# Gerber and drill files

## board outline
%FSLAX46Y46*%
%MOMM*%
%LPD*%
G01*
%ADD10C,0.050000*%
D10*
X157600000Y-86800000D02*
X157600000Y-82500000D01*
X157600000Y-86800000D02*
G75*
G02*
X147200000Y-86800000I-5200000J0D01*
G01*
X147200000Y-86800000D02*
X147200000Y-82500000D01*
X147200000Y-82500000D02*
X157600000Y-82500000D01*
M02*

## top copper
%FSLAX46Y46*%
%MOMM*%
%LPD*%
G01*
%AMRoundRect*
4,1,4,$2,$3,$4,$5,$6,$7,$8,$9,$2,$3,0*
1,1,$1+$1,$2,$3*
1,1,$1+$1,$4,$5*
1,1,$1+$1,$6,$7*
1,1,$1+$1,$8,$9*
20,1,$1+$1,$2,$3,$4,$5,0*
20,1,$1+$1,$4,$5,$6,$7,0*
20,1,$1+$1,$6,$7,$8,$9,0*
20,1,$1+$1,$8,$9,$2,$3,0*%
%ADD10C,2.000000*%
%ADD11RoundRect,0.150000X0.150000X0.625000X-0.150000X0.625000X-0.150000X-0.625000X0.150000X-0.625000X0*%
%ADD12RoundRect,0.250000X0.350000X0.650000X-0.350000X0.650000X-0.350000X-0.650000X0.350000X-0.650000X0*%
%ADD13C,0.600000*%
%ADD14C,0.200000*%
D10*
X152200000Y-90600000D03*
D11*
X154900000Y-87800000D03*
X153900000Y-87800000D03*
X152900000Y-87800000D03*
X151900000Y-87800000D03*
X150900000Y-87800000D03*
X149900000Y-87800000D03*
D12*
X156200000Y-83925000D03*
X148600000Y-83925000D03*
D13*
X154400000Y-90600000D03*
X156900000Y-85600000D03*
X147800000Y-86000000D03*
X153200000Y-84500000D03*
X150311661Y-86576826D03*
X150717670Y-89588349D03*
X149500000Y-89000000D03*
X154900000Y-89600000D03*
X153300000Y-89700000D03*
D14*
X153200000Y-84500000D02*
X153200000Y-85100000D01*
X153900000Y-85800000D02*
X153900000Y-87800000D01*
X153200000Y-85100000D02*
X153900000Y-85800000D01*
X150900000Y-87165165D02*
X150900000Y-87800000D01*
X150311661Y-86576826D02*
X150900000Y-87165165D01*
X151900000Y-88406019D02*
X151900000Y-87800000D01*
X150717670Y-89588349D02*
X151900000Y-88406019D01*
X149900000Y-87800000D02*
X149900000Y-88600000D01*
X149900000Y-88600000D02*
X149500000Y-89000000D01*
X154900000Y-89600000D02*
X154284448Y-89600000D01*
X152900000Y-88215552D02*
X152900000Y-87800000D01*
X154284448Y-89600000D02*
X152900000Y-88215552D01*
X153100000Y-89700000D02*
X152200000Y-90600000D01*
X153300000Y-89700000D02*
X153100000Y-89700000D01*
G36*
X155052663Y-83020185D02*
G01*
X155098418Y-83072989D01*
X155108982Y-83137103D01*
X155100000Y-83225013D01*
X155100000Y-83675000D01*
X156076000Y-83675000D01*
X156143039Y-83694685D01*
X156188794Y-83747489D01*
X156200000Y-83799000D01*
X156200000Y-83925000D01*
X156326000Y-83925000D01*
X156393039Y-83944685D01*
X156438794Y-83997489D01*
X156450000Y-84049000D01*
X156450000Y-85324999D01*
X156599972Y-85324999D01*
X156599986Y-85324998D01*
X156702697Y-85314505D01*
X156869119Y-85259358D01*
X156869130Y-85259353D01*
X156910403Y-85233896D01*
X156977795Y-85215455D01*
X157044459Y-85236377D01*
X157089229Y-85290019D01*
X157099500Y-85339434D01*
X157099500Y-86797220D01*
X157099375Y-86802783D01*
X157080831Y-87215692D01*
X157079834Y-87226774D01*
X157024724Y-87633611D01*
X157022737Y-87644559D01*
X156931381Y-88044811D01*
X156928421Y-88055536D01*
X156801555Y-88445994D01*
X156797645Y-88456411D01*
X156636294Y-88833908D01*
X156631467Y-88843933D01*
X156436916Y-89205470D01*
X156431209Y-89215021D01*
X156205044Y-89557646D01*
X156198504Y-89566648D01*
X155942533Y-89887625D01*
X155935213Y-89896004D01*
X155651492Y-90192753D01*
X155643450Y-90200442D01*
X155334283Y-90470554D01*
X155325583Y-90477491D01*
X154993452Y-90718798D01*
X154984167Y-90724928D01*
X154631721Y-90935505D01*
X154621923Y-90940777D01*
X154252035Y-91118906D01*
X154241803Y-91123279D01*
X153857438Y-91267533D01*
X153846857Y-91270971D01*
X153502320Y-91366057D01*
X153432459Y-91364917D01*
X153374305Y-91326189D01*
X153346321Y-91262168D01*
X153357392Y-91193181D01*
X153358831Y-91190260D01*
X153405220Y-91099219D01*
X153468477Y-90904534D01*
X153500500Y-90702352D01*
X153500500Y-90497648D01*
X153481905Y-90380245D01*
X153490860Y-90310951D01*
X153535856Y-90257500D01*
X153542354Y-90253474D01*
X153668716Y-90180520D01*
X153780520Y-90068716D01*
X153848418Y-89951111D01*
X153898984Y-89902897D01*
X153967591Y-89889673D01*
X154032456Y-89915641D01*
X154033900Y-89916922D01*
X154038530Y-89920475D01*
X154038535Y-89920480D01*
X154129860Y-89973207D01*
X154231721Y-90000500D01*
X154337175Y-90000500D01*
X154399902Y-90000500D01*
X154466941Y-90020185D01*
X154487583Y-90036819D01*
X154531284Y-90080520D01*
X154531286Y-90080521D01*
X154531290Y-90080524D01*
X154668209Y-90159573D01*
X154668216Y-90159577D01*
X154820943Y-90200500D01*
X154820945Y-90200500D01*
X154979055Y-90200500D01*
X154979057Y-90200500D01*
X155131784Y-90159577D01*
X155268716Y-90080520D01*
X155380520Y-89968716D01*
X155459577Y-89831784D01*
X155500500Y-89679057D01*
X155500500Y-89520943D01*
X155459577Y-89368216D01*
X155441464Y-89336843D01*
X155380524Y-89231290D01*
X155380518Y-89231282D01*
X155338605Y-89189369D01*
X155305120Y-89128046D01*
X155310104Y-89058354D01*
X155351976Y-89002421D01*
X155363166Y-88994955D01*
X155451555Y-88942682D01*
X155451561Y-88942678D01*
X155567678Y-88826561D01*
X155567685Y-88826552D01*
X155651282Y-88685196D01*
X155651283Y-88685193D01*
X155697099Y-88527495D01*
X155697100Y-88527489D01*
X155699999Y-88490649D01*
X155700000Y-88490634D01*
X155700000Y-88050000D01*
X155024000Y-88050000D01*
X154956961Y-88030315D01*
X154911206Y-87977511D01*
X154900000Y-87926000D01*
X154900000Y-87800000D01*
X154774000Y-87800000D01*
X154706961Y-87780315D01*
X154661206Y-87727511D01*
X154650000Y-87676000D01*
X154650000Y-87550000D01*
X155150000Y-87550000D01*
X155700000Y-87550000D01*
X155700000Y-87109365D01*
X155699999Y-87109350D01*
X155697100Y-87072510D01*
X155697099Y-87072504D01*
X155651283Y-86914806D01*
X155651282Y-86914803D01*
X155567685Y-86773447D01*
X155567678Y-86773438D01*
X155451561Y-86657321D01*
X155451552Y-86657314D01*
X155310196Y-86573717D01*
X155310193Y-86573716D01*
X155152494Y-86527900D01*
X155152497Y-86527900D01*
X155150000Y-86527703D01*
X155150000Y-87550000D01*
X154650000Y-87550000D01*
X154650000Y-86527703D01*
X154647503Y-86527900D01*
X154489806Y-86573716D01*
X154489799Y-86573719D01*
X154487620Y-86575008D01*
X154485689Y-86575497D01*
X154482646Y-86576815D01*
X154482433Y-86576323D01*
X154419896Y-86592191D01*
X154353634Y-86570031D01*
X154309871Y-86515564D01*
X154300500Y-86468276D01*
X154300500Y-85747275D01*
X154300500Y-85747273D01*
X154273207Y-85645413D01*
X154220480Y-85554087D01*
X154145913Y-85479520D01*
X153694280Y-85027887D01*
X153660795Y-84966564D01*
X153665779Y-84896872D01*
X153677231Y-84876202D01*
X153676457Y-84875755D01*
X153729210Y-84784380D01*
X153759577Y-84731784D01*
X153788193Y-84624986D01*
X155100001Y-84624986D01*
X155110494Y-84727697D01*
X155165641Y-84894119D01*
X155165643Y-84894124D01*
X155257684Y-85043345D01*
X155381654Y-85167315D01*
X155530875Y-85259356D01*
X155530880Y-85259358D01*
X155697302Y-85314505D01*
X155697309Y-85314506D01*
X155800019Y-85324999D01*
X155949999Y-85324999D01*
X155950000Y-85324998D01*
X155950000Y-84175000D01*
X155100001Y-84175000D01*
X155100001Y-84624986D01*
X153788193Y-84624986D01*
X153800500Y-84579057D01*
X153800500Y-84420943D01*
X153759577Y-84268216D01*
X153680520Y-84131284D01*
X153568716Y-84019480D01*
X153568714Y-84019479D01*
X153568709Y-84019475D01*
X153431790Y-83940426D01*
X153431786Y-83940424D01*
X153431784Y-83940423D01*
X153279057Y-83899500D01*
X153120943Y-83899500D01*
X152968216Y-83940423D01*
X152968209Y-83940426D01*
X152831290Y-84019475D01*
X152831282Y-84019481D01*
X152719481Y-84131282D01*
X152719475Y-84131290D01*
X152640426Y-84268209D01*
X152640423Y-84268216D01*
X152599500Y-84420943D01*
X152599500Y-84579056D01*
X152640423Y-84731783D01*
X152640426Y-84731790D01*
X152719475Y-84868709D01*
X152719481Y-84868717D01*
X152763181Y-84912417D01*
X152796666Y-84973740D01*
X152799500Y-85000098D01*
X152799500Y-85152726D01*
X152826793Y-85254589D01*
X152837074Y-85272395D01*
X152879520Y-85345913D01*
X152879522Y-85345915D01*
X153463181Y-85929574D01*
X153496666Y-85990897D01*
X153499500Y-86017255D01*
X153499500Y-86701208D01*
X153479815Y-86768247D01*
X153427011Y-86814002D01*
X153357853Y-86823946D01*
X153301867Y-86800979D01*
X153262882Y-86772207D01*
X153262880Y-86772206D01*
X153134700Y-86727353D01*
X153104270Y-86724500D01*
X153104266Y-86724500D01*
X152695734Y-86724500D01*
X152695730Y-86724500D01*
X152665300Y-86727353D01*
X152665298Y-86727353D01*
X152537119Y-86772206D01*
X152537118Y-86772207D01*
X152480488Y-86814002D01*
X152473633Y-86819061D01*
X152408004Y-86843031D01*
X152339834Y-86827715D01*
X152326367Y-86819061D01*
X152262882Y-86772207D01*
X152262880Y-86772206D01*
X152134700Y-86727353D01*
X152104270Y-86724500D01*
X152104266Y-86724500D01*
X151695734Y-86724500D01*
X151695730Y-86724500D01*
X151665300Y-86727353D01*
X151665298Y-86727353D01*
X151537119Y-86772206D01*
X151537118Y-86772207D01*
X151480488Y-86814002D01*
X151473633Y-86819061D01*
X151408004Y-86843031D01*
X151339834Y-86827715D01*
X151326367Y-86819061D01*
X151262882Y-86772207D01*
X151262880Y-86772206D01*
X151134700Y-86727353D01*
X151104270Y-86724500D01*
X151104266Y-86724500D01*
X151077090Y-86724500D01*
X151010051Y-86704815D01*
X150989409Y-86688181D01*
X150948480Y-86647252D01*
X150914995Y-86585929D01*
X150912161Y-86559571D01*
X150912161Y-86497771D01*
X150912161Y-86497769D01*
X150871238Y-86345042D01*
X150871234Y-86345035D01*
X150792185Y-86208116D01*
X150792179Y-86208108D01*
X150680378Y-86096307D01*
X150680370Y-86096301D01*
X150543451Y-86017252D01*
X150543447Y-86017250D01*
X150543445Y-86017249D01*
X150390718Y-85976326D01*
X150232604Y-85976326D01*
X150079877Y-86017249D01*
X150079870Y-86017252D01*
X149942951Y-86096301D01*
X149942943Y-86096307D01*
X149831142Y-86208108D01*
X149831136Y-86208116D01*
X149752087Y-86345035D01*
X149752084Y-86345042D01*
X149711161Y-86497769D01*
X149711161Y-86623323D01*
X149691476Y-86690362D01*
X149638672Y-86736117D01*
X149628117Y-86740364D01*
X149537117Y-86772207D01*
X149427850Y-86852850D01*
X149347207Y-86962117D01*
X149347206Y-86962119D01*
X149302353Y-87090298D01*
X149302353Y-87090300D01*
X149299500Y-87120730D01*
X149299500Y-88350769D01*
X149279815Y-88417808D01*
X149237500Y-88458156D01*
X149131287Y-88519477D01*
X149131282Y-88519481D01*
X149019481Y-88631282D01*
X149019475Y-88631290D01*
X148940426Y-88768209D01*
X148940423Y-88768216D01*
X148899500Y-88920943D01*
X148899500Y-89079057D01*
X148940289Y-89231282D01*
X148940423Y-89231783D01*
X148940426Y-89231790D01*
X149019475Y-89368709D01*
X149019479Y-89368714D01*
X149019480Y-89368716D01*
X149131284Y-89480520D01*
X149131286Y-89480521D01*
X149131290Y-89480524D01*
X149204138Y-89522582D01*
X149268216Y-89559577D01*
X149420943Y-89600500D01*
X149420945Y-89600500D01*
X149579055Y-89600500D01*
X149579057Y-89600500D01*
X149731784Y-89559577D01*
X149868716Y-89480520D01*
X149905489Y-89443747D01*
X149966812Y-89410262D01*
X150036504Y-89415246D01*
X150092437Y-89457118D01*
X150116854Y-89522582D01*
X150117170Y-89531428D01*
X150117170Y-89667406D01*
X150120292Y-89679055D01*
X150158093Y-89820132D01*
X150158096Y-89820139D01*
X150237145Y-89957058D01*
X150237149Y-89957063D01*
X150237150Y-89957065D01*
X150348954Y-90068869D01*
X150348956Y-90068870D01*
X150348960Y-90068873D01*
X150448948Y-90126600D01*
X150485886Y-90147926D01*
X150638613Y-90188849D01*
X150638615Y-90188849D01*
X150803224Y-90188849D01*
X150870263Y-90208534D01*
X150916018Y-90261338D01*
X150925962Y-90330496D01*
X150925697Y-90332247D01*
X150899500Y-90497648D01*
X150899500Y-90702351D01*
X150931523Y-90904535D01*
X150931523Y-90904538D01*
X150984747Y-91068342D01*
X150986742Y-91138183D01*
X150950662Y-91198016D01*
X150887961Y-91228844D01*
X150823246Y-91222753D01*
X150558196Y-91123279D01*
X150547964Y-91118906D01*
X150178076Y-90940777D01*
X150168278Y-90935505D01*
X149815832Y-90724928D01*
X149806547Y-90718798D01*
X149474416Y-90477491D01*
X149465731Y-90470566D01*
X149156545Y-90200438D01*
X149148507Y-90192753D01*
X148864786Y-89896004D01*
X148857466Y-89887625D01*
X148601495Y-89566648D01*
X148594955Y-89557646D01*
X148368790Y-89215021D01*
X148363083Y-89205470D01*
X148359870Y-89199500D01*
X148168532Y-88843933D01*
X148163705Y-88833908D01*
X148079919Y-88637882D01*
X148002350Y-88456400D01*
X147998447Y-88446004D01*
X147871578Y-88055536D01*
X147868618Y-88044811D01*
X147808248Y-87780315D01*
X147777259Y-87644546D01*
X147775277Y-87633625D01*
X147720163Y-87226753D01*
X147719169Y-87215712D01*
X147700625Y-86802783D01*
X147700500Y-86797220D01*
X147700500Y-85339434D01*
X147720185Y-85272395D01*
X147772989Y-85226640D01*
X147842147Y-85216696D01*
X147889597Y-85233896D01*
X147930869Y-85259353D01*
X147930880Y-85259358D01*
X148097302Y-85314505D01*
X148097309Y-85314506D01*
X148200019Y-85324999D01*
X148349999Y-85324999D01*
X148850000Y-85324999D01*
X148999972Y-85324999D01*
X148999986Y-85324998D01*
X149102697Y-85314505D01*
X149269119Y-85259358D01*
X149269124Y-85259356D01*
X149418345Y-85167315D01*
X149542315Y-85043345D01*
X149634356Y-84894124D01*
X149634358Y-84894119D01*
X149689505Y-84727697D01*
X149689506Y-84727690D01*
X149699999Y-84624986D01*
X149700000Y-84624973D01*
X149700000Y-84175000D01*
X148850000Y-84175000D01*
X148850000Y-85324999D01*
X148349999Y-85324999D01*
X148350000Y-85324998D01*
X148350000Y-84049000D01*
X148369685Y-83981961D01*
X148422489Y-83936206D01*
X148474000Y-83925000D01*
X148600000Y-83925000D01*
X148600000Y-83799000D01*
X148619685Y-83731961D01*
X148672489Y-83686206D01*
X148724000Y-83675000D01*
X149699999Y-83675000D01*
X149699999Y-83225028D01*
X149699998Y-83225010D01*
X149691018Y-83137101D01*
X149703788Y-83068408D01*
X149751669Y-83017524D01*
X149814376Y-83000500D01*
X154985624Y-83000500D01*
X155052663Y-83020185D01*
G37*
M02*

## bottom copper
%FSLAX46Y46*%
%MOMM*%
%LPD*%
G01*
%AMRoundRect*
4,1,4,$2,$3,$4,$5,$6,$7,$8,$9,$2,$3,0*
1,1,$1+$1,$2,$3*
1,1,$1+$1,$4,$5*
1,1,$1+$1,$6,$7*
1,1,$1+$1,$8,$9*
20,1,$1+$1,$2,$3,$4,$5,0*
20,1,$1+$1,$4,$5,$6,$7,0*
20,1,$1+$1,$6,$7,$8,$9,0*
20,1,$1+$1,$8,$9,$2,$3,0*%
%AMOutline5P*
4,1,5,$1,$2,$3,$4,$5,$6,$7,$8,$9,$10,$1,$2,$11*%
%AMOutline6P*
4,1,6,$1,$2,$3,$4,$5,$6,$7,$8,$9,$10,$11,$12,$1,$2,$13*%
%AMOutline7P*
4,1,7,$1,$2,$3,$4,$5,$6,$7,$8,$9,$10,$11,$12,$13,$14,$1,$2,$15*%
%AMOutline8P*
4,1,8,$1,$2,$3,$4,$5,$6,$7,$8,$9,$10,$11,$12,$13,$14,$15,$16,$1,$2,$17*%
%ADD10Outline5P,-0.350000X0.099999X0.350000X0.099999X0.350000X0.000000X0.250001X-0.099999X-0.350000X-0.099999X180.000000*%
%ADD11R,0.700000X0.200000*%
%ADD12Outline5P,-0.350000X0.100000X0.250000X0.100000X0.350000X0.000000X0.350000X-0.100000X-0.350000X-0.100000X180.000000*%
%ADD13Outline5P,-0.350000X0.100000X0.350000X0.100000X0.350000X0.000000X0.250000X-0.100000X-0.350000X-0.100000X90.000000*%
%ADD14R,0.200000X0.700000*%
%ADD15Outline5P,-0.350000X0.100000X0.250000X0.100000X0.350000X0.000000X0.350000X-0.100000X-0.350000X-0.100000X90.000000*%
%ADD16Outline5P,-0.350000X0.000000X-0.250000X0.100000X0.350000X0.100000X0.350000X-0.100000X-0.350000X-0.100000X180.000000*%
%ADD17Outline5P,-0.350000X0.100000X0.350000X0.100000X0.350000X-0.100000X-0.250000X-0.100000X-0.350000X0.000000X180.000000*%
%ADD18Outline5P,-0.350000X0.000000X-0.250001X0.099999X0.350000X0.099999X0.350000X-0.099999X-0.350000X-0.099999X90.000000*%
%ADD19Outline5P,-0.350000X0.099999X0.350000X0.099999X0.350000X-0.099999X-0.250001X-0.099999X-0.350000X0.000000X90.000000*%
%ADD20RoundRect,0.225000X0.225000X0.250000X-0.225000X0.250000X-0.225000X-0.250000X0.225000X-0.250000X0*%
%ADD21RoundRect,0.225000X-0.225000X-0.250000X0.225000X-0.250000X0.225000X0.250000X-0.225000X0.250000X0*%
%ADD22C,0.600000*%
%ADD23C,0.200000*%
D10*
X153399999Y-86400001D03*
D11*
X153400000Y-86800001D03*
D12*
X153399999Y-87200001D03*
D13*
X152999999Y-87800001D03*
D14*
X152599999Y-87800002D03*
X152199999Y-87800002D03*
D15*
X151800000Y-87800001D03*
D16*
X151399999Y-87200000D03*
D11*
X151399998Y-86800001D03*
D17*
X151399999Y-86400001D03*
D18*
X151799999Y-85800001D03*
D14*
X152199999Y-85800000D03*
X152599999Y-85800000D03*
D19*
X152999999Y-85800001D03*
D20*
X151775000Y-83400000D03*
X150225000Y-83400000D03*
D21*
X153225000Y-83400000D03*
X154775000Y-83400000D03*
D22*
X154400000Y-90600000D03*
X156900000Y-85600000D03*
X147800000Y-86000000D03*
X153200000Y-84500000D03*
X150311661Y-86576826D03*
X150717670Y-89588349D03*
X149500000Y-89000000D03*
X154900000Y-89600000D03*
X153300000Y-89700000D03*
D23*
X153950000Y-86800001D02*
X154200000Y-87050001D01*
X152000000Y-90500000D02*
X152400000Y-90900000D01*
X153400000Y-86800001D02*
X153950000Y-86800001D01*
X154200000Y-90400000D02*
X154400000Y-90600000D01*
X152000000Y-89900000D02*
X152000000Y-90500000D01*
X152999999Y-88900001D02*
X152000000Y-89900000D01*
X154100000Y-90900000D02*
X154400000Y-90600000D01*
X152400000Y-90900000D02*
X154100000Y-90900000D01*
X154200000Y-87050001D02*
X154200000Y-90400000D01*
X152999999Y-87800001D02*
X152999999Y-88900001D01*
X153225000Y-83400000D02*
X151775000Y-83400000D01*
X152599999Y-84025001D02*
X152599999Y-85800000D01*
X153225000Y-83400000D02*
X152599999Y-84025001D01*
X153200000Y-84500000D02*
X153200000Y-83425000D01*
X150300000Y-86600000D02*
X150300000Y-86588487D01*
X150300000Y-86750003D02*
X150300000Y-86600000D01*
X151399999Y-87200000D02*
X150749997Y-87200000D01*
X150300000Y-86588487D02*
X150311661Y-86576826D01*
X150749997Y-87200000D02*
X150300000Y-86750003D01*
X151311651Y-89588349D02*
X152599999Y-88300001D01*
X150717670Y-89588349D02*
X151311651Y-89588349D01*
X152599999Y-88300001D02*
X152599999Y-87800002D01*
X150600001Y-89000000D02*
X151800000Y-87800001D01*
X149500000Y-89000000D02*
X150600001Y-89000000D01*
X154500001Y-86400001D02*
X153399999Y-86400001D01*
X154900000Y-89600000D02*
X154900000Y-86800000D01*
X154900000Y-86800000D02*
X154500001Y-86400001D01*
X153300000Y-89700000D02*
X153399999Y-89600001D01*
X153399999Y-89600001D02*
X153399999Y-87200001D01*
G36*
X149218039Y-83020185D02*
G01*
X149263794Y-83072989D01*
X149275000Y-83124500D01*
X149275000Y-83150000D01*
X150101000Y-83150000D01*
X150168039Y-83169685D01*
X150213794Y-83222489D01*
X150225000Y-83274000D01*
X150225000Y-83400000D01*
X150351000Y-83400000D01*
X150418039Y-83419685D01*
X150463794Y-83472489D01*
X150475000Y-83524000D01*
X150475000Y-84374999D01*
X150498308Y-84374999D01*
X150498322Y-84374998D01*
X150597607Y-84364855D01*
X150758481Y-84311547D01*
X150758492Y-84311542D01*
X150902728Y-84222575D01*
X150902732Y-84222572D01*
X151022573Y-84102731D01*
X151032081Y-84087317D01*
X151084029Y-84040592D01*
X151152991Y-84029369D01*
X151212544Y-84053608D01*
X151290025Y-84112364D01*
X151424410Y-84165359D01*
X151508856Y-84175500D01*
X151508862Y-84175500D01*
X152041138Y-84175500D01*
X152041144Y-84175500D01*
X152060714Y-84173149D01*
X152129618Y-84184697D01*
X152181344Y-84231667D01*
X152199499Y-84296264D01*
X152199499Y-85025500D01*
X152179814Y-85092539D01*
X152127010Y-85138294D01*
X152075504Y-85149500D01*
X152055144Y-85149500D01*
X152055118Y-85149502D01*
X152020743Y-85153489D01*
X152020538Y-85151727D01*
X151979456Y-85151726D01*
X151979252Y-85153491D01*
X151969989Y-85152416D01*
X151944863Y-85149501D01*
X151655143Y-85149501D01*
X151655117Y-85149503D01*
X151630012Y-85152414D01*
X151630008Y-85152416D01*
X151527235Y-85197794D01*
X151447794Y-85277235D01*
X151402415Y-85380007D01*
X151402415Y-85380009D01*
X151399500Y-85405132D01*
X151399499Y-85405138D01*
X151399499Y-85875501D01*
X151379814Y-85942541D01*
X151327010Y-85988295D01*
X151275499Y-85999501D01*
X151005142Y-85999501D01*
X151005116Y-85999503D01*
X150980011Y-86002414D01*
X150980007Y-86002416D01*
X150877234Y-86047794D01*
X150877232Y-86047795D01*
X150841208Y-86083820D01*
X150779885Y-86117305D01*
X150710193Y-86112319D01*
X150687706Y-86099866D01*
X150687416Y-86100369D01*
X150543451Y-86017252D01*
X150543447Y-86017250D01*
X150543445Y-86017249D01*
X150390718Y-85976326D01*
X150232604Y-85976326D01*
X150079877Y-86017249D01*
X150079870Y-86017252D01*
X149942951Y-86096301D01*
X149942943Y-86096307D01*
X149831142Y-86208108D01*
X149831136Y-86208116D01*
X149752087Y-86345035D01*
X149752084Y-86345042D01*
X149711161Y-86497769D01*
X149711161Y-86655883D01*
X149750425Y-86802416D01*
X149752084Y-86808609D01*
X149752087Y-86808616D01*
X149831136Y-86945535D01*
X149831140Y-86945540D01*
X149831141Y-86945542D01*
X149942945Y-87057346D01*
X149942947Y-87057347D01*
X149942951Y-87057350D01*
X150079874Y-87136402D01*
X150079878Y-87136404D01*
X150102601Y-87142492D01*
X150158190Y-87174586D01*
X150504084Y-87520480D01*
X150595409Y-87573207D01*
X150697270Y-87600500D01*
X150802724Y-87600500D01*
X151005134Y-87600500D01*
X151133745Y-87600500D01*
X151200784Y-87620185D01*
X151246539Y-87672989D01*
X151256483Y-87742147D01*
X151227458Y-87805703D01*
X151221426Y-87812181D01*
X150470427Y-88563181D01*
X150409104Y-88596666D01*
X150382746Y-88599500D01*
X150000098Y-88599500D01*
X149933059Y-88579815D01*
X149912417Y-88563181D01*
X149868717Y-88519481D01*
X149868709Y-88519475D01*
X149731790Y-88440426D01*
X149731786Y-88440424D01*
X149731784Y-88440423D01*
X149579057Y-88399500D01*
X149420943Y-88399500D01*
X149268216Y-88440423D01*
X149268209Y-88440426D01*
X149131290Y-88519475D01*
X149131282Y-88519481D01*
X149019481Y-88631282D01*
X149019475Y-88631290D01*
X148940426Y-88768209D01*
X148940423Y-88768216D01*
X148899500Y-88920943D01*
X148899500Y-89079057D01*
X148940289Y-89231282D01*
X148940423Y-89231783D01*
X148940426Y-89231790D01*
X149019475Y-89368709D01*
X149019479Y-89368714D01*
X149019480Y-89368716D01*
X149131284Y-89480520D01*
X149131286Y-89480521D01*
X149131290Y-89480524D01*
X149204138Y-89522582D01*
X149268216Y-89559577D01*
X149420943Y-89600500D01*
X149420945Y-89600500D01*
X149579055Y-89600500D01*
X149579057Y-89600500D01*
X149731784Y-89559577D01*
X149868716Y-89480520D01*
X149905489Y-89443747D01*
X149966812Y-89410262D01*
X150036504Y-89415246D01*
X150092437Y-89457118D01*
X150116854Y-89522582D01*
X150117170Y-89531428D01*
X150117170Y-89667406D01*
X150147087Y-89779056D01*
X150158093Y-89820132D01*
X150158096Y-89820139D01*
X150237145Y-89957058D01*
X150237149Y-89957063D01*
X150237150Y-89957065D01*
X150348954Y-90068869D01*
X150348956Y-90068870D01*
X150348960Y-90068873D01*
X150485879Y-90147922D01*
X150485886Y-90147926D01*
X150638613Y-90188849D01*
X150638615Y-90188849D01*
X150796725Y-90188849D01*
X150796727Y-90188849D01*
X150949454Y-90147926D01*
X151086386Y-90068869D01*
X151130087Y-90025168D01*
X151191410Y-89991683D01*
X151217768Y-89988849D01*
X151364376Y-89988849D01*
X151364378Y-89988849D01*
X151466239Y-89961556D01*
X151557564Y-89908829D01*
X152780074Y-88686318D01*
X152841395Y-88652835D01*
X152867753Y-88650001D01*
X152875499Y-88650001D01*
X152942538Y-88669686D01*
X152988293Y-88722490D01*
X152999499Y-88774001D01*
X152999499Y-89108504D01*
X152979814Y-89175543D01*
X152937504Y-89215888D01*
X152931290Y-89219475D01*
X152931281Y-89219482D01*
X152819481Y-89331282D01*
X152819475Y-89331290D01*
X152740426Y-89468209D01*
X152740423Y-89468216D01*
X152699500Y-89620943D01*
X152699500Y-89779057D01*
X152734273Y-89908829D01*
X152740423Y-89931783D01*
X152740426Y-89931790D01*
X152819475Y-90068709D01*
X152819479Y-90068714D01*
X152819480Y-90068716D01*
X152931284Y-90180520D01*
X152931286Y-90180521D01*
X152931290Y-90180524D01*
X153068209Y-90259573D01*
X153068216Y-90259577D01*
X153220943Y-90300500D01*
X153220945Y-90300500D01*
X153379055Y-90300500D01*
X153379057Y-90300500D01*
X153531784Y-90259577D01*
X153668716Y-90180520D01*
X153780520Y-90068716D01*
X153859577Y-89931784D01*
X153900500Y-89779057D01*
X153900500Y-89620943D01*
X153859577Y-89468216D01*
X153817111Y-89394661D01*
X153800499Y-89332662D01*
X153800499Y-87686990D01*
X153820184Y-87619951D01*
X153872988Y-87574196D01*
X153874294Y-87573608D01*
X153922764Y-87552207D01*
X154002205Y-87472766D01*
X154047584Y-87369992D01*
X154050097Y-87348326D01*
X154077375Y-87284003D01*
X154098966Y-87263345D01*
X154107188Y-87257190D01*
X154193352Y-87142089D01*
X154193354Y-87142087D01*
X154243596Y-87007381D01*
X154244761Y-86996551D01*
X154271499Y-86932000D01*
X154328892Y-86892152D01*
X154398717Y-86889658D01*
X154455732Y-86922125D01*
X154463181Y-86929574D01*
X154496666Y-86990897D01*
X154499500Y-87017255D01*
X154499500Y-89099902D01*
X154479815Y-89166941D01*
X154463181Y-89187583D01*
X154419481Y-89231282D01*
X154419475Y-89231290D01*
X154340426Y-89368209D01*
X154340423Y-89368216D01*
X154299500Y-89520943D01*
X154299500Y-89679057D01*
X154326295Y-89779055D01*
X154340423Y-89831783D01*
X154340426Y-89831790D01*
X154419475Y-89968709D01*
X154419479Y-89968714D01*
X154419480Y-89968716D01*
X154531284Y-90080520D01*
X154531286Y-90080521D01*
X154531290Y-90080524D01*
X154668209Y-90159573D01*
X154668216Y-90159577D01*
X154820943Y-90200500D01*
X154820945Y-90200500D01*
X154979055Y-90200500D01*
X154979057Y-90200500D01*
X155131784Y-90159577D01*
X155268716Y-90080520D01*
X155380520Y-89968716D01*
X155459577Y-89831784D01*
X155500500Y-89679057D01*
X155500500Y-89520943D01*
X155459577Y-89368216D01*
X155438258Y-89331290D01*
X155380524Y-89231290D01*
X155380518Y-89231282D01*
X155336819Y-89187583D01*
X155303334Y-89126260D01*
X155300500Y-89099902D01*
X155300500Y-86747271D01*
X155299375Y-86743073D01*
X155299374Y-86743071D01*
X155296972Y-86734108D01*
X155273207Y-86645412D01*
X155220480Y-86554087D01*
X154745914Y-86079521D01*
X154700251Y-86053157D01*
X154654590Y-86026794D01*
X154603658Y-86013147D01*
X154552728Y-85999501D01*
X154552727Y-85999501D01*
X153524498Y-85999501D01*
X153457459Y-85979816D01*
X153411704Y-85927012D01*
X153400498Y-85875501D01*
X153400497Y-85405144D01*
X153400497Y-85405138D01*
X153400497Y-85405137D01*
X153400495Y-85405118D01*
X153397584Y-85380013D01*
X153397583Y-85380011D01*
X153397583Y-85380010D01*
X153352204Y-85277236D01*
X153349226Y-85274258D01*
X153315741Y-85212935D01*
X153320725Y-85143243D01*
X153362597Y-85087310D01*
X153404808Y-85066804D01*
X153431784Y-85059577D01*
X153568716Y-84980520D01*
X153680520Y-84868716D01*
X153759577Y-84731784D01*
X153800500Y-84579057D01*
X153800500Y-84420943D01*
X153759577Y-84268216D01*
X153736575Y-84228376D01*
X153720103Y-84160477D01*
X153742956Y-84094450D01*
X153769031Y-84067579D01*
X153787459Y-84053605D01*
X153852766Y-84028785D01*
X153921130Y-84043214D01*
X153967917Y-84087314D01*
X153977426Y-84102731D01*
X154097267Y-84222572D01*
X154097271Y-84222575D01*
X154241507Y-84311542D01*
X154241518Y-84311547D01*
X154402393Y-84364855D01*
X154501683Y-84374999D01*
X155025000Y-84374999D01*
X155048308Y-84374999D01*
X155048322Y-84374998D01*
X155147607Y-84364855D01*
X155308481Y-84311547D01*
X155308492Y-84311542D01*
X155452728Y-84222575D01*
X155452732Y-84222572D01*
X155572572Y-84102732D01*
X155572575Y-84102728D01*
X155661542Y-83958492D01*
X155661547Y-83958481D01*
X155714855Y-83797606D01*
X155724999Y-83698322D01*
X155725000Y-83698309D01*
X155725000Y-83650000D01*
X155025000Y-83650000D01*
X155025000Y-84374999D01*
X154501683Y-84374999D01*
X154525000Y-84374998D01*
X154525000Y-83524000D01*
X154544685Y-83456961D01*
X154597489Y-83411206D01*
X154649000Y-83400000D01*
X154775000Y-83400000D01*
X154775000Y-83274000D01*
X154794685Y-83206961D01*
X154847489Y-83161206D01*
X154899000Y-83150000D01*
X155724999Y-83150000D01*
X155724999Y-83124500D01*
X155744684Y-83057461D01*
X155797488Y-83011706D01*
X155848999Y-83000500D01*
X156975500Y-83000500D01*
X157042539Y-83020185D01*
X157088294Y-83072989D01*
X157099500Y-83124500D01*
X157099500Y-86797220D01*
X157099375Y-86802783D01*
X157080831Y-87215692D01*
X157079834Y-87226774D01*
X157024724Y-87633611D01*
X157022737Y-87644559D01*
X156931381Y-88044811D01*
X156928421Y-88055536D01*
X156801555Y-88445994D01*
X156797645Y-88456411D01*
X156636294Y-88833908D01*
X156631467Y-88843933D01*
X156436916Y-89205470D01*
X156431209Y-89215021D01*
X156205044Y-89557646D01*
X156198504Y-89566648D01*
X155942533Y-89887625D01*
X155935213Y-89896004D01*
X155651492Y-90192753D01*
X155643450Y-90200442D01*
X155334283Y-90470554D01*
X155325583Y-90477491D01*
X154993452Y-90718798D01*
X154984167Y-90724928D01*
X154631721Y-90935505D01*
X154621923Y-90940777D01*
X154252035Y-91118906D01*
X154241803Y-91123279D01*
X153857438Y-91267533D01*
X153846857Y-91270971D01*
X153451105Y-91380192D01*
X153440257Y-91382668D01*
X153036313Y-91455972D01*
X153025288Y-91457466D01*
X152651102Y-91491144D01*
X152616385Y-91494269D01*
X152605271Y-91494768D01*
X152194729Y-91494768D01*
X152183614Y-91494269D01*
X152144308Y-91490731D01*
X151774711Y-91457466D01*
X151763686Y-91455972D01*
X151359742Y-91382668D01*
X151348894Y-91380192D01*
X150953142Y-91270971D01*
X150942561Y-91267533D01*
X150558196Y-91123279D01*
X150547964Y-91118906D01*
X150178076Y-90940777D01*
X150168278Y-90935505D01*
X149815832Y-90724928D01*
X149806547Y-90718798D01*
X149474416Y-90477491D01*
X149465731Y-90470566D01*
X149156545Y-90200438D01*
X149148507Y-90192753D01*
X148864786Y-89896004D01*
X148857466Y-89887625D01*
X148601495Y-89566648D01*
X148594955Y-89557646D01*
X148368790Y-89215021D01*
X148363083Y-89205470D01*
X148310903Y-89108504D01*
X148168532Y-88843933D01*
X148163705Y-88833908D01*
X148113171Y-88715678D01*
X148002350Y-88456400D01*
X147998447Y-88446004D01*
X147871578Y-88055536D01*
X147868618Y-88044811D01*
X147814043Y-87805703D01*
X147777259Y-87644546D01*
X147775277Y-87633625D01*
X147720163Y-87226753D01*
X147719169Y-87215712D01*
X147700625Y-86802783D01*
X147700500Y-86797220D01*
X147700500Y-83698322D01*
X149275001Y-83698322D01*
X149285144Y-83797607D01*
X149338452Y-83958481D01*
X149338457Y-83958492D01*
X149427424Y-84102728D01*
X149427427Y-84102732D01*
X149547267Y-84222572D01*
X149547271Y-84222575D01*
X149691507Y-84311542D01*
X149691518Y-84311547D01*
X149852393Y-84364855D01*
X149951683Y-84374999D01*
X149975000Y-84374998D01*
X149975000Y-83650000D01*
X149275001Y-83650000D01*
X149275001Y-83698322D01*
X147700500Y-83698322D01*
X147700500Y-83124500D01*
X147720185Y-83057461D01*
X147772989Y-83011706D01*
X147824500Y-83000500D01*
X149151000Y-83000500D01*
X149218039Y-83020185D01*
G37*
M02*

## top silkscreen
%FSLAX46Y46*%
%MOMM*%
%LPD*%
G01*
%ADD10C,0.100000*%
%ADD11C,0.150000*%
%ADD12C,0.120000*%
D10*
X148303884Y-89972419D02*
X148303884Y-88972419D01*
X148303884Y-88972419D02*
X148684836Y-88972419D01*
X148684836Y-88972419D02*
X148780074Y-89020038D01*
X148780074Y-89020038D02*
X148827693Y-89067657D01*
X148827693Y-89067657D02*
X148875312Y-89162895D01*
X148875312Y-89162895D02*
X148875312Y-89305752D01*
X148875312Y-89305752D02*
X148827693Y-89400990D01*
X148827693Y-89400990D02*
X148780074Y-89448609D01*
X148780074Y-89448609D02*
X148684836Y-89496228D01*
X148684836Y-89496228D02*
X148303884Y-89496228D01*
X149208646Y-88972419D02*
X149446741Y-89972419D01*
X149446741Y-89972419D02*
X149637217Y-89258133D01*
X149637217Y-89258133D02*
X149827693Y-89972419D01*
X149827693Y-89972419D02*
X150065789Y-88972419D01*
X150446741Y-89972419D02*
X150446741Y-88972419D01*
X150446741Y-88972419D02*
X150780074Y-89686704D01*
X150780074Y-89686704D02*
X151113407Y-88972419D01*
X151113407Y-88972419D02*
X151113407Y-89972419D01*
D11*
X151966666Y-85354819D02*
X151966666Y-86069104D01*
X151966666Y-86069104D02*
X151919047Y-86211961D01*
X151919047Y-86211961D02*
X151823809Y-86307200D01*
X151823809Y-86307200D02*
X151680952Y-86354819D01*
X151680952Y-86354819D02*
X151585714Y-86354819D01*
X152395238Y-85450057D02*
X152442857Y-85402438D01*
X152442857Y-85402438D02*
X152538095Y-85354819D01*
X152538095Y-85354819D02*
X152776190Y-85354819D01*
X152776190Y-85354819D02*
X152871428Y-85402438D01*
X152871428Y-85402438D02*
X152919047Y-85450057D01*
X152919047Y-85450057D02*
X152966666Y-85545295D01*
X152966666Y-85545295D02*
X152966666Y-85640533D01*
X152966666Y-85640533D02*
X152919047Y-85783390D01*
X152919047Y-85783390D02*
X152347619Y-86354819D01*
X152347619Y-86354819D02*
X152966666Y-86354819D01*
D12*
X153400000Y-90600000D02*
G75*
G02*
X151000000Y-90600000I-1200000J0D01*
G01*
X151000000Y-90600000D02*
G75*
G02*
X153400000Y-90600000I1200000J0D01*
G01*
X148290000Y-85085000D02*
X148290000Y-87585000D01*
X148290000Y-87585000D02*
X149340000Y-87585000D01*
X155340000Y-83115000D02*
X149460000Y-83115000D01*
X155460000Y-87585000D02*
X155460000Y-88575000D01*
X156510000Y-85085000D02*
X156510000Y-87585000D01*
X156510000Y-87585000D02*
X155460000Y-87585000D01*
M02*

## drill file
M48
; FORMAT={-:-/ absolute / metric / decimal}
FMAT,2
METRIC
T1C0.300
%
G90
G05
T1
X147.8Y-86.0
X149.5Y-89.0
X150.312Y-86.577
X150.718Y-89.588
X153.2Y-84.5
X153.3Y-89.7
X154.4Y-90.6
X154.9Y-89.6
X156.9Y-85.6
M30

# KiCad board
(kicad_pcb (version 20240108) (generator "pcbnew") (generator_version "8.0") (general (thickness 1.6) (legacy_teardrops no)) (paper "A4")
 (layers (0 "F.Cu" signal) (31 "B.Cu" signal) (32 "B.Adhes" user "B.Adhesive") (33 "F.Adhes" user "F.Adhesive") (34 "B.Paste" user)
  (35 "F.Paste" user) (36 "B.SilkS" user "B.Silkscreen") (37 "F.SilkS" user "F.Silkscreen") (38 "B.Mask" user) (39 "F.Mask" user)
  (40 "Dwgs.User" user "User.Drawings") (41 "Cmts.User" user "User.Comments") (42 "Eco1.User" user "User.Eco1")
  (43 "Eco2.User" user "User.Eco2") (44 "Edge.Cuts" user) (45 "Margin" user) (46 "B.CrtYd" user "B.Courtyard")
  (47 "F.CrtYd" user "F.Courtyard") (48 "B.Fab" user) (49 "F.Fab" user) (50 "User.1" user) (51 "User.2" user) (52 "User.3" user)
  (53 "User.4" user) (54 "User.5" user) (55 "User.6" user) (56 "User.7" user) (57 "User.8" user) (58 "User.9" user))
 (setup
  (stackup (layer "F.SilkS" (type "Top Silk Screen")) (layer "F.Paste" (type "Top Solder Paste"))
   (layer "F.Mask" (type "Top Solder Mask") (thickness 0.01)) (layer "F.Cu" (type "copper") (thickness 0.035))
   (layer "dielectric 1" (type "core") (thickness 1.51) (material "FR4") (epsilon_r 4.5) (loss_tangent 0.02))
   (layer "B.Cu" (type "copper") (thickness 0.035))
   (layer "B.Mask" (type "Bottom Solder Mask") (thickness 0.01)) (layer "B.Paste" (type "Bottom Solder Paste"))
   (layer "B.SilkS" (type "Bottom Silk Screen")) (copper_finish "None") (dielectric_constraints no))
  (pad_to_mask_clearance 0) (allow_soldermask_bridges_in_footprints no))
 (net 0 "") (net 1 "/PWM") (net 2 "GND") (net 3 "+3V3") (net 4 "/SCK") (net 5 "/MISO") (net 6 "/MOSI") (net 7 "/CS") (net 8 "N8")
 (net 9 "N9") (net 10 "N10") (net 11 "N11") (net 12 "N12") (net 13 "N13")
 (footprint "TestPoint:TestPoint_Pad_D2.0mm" (layer "F.Cu") (at 152.2 90.6)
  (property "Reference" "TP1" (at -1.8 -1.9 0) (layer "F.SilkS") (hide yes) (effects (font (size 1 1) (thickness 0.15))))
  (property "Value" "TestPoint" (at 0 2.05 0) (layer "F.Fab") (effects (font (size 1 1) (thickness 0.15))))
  (fp_circle (center 0 0) (end 0 1.2) (stroke (width 0.12) (type solid)) (fill none) (layer "F.SilkS"))
  (pad "1" smd circle (at 0 0) (size 2 2) (layers "F.Cu" "F.Mask") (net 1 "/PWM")))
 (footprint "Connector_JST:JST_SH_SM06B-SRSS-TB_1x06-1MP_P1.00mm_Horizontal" (layer "F.Cu") (at 152.4 85.8 180)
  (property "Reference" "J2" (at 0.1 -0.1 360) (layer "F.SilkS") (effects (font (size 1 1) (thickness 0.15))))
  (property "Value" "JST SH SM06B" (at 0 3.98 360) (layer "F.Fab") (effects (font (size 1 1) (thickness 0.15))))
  (fp_line (start 4.11 0.715) (end 4.11 -1.785) (stroke (width 0.12) (type solid)) (layer "F.SilkS"))
  (fp_line (start 4.11 -1.785) (end 3.06 -1.785) (stroke (width 0.12) (type solid)) (layer "F.SilkS"))
  (fp_line (start -2.94 2.685) (end 2.94 2.685) (stroke (width 0.12) (type solid)) (layer "F.SilkS"))
  (fp_line (start -3.06 -1.785) (end -3.06 -2.775) (stroke (width 0.12) (type solid)) (layer "F.SilkS"))
  (fp_line (start -4.11 0.715) (end -4.11 -1.785) (stroke (width 0.12) (type solid)) (layer "F.SilkS"))
  (fp_line (start -4.11 -1.785) (end -3.06 -1.785) (stroke (width 0.12) (type solid)) (layer "F.SilkS"))
  (pad "1" smd roundrect (at -2.5 -2 180) (size 0.6 1.55) (layers "F.Cu" "F.Paste" "F.Mask") (roundrect_rratio 0.25) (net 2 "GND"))
  (pad "2" smd roundrect (at -1.5 -2 180) (size 0.6 1.55) (layers "F.Cu" "F.Paste" "F.Mask") (roundrect_rratio 0.25) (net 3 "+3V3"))
  (pad "3" smd roundrect (at -0.5 -2 180) (size 0.6 1.55) (layers "F.Cu" "F.Paste" "F.Mask") (roundrect_rratio 0.25) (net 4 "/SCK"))
  (pad "4" smd roundrect (at 0.5 -2 180) (size 0.6 1.55) (layers "F.Cu" "F.Paste" "F.Mask") (roundrect_rratio 0.25) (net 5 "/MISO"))
  (pad "5" smd roundrect (at 1.5 -2 180) (size 0.6 1.55) (layers "F.Cu" "F.Paste" "F.Mask") (roundrect_rratio 0.25) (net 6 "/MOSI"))
  (pad "6" smd roundrect (at 2.5 -2 180) (size 0.6 1.55) (layers "F.Cu" "F.Paste" "F.Mask") (roundrect_rratio 0.25) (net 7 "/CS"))
  (pad "MP" smd roundrect (at -3.8 1.875 180) (size 1.2 1.8) (layers "F.Cu" "F.Paste" "F.Mask") (roundrect_rratio 0.208333) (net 2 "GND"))
  (pad "MP" smd roundrect (at 3.8 1.875 180) (size 1.2 1.8) (layers "F.Cu" "F.Paste" "F.Mask") (roundrect_rratio 0.208333) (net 2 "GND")))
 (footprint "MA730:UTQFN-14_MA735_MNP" (layer "B.Cu") (at 152.399999 86.800001 180)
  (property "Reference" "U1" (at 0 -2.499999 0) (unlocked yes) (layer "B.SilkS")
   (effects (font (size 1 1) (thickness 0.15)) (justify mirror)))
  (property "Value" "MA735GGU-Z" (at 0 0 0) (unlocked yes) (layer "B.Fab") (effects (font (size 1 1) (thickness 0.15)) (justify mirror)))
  (pad "1" smd roundrect (at -1 0.4 180) (size 0.7 0.199998) (layers "B.Cu" "B.Paste" "B.Mask") (roundrect_rratio 0) (chamfer_ratio 0.5)
   (chamfer bottom_right) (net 4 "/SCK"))
  (pad "2" smd rect (at -1.000001 0 180) (size 0.7 0.2) (layers "B.Cu" "B.Paste" "B.Mask") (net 2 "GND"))
  (pad "3" smd roundrect (at -1 -0.4 180) (size 0.7 0.2) (layers "B.Cu" "B.Paste" "B.Mask") (roundrect_rratio 0) (chamfer_ratio 0.5)
   (chamfer top_right) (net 1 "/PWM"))
  (pad "4" smd roundrect (at -0.6 -1 90) (size 0.7 0.2) (layers "B.Cu" "B.Paste" "B.Mask") (roundrect_rratio 0) (chamfer_ratio 0.5)
   (chamfer bottom_right) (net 2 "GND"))
  (pad "5" smd rect (at -0.2 -1.000001 90) (size 0.7 0.2) (layers "B.Cu" "B.Paste" "B.Mask") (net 5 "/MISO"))
  (pad "6" smd rect (at 0.2 -1.000001 90) (size 0.7 0.2) (layers "B.Cu" "B.Paste" "B.Mask") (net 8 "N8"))
  (pad "7" smd roundrect (at 0.599999 -1 90) (size 0.7 0.199999) (layers "B.Cu" "B.Paste" "B.Mask") (roundrect_rratio 0) (chamfer_ratio 0.5)
   (chamfer top_right) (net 7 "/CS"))
  (pad "8" smd roundrect (at 1 -0.399999 180) (size 0.7 0.2) (layers "B.Cu" "B.Paste" "B.Mask") (roundrect_rratio 0) (chamfer_ratio 0.5)
   (chamfer top_left) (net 6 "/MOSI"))
  (pad "9" smd rect (at 1.000001 0 180) (size 0.7 0.2) (layers "B.Cu" "B.Paste" "B.Mask") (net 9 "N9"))
  (pad "10" smd roundrect (at 1 0.4 180) (size 0.7 0.2) (layers "B.Cu" "B.Paste" "B.Mask") (roundrect_rratio 0) (chamfer_ratio 0.5)
   (chamfer bottom_left) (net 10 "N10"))
  (pad "11" smd roundrect (at 0.6 1 90) (size 0.7 0.199998) (layers "B.Cu" "B.Paste" "B.Mask") (roundrect_rratio 0) (chamfer_ratio 0.5)
   (chamfer top_left) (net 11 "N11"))
  (pad "12" smd rect (at 0.2 1.000001 90) (size 0.7 0.2) (layers "B.Cu" "B.Paste" "B.Mask") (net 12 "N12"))
  (pad "13" smd rect (at -0.2 1.000001 90) (size 0.7 0.2) (layers "B.Cu" "B.Paste" "B.Mask") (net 3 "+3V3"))
  (pad "14" smd roundrect (at -0.6 1 90) (size 0.7 0.199998) (layers "B.Cu" "B.Paste" "B.Mask") (roundrect_rratio 0) (chamfer_ratio 0.5)
   (chamfer bottom_left) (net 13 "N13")))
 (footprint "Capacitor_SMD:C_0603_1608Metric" (layer "B.Cu") (at 151 83.4 180)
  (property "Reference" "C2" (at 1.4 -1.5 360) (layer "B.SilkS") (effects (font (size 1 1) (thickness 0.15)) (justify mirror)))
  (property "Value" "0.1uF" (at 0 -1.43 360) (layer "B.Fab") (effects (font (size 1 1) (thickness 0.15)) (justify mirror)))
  (pad "1" smd roundrect (at -0.775 0 180) (size 0.9 0.95) (layers "B.Cu" "B.Paste" "B.Mask") (roundrect_rratio 0.25) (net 3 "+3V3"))
  (pad "2" smd roundrect (at 0.775 0 180) (size 0.9 0.95) (layers "B.Cu" "B.Paste" "B.Mask") (roundrect_rratio 0.25) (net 2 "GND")))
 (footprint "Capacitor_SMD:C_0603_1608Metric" (layer "B.Cu") (at 154 83.4)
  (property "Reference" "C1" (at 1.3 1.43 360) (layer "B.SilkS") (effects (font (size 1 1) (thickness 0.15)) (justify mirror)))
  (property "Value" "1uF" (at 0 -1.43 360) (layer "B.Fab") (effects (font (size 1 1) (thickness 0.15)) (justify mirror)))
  (pad "1" smd roundrect (at -0.775 0) (size 0.9 0.95) (layers "B.Cu" "B.Paste" "B.Mask") (roundrect_rratio 0.25) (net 3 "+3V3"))
  (pad "2" smd roundrect (at 0.775 0) (size 0.9 0.95) (layers "B.Cu" "B.Paste" "B.Mask") (roundrect_rratio 0.25) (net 2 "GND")))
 (gr_line (start 157.6 86.8) (end 157.6 82.5) (stroke (width 0.05) (type default)) (layer "Edge.Cuts"))
 (gr_arc (start 157.6 86.8) (mid 152.4 92) (end 147.2 86.8) (stroke (width 0.05) (type default)) (layer "Edge.Cuts"))
 (gr_line (start 147.2 86.8) (end 147.2 82.5) (stroke (width 0.05) (type default)) (layer "Edge.Cuts"))
 (gr_line (start 147.2 82.5) (end 157.6 82.5) (stroke (width 0.05) (type default)) (layer "Edge.Cuts"))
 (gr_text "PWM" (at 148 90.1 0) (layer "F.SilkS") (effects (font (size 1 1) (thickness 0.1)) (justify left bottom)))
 (via (at 154.4 90.6) (size 0.6) (drill 0.3) (layers "F.Cu" "B.Cu") (free yes) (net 2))
 (via (at 156.9 85.6) (size 0.6) (drill 0.3) (layers "F.Cu" "B.Cu") (free yes) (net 2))
 (via (at 147.8 86) (size 0.6) (drill 0.3) (layers "F.Cu" "B.Cu") (free yes) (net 2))
 (segment (start 153.95 86.800001) (end 154.2 87.050001) (width 0.2) (layer "B.Cu") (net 2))
 (segment (start 152 90.5) (end 152.4 90.9) (width 0.2) (layer "B.Cu") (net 2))
 (segment (start 153.4 86.800001) (end 153.95 86.800001) (width 0.2) (layer "B.Cu") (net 2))
 (segment (start 154.2 90.4) (end 154.4 90.6) (width 0.2) (layer "B.Cu") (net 2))
 (segment (start 152 89.9) (end 152 90.5) (width 0.2) (layer "B.Cu") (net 2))
 (segment (start 152.999999 88.900001) (end 152 89.9) (width 0.2) (layer "B.Cu") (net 2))
 (segment (start 154.1 90.9) (end 154.4 90.6) (width 0.2) (layer "B.Cu") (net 2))
 (segment (start 152.4 90.9) (end 154.1 90.9) (width 0.2) (layer "B.Cu") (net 2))
 (segment (start 154.2 87.050001) (end 154.2 90.4) (width 0.2) (layer "B.Cu") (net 2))
 (segment (start 152.999999 87.800001) (end 152.999999 88.900001) (width 0.2) (layer "B.Cu") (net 2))
 (segment (start 153.2 84.5) (end 153.2 85.1) (width 0.2) (layer "F.Cu") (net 3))
 (segment (start 153.9 85.8) (end 153.9 87.8) (width 0.2) (layer "F.Cu") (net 3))
 (segment (start 153.2 85.1) (end 153.9 85.8) (width 0.2) (layer "F.Cu") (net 3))
 (via (at 153.2 84.5) (size 0.6) (drill 0.3) (layers "F.Cu" "B.Cu") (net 3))
 (segment (start 153.225 83.4) (end 151.775 83.4) (width 0.2) (layer "B.Cu") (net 3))
 (segment (start 152.599999 84.025001) (end 152.599999 85.8) (width 0.2) (layer "B.Cu") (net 3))
 (segment (start 153.225 83.4) (end 152.599999 84.025001) (width 0.2) (layer "B.Cu") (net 3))
 (segment (start 153.2 84.5) (end 153.2 83.425) (width 0.2) (layer "B.Cu") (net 3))
 (segment (start 150.9 87.165165) (end 150.9 87.8) (width 0.2) (layer "F.Cu") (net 6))
 (segment (start 150.311661 86.576826) (end 150.9 87.165165) (width 0.2) (layer "F.Cu") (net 6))
 (via (at 150.311661 86.576826) (size 0.6) (drill 0.3) (layers "F.Cu" "B.Cu") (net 6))
 (segment (start 150.3 86.6) (end 150.3 86.588487) (width 0.2) (layer "B.Cu") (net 6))
 (segment (start 150.3 86.750003) (end 150.3 86.6) (width 0.2) (layer "B.Cu") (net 6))
 (segment (start 151.399999 87.2) (end 150.749997 87.2) (width 0.2) (layer "B.Cu") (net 6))
 (segment (start 150.3 86.588487) (end 150.311661 86.576826) (width 0.2) (layer "B.Cu") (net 6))
 (segment (start 150.749997 87.2) (end 150.3 86.750003) (width 0.2) (layer "B.Cu") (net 6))
 (segment (start 151.9 88.406019) (end 151.9 87.8) (width 0.2) (layer "F.Cu") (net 5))
 (segment (start 150.71767 89.588349) (end 151.9 88.406019) (width 0.2) (layer "F.Cu") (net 5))
 (via (at 150.71767 89.588349) (size 0.6) (drill 0.3) (layers "F.Cu" "B.Cu") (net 5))
 (segment (start 151.311651 89.588349) (end 152.599999 88.300001) (width 0.2) (layer "B.Cu") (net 5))
 (segment (start 150.71767 89.588349) (end 151.311651 89.588349) (width 0.2) (layer "B.Cu") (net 5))
 (segment (start 152.599999 88.300001) (end 152.599999 87.800002) (width 0.2) (layer "B.Cu") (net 5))
 (segment (start 149.9 87.8) (end 149.9 88.6) (width 0.2) (layer "F.Cu") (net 7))
 (segment (start 149.9 88.6) (end 149.5 89) (width 0.2) (layer "F.Cu") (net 7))
 (via (at 149.5 89) (size 0.6) (drill 0.3) (layers "F.Cu" "B.Cu") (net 7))
 (segment (start 150.600001 89) (end 151.8 87.800001) (width 0.2) (layer "B.Cu") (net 7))
 (segment (start 149.5 89) (end 150.600001 89) (width 0.2) (layer "B.Cu") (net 7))
 (segment (start 154.9 89.6) (end 154.284448 89.6) (width 0.2) (layer "F.Cu") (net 4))
 (segment (start 152.9 88.215552) (end 152.9 87.8) (width 0.2) (layer "F.Cu") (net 4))
 (segment (start 154.284448 89.6) (end 152.9 88.215552) (width 0.2) (layer "F.Cu") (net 4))
 (via (at 154.9 89.6) (size 0.6) (drill 0.3) (layers "F.Cu" "B.Cu") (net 4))
 (segment (start 154.500001 86.400001) (end 153.399999 86.400001) (width 0.2) (layer "B.Cu") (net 4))
 (segment (start 154.9 89.6) (end 154.9 86.8) (width 0.2) (layer "B.Cu") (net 4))
 (segment (start 154.9 86.8) (end 154.500001 86.400001) (width 0.2) (layer "B.Cu") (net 4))
 (segment (start 153.1 89.7) (end 152.2 90.6) (width 0.2) (layer "F.Cu") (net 1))
 (segment (start 153.3 89.7) (end 153.1 89.7) (width 0.2) (layer "F.Cu") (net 1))
 (via (at 153.3 89.7) (size 0.6) (drill 0.3) (layers "F.Cu" "B.Cu") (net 1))
 (segment (start 153.3 89.7) (end 153.399999 89.600001) (width 0.2) (layer "B.Cu") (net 1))
 (segment (start 153.399999 89.600001) (end 153.399999 87.200001) (width 0.2) (layer "B.Cu") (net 1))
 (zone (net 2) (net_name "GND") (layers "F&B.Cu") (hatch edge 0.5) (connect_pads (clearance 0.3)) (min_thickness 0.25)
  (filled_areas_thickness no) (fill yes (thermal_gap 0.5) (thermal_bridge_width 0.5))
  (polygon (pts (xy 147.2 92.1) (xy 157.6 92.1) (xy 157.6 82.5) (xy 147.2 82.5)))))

